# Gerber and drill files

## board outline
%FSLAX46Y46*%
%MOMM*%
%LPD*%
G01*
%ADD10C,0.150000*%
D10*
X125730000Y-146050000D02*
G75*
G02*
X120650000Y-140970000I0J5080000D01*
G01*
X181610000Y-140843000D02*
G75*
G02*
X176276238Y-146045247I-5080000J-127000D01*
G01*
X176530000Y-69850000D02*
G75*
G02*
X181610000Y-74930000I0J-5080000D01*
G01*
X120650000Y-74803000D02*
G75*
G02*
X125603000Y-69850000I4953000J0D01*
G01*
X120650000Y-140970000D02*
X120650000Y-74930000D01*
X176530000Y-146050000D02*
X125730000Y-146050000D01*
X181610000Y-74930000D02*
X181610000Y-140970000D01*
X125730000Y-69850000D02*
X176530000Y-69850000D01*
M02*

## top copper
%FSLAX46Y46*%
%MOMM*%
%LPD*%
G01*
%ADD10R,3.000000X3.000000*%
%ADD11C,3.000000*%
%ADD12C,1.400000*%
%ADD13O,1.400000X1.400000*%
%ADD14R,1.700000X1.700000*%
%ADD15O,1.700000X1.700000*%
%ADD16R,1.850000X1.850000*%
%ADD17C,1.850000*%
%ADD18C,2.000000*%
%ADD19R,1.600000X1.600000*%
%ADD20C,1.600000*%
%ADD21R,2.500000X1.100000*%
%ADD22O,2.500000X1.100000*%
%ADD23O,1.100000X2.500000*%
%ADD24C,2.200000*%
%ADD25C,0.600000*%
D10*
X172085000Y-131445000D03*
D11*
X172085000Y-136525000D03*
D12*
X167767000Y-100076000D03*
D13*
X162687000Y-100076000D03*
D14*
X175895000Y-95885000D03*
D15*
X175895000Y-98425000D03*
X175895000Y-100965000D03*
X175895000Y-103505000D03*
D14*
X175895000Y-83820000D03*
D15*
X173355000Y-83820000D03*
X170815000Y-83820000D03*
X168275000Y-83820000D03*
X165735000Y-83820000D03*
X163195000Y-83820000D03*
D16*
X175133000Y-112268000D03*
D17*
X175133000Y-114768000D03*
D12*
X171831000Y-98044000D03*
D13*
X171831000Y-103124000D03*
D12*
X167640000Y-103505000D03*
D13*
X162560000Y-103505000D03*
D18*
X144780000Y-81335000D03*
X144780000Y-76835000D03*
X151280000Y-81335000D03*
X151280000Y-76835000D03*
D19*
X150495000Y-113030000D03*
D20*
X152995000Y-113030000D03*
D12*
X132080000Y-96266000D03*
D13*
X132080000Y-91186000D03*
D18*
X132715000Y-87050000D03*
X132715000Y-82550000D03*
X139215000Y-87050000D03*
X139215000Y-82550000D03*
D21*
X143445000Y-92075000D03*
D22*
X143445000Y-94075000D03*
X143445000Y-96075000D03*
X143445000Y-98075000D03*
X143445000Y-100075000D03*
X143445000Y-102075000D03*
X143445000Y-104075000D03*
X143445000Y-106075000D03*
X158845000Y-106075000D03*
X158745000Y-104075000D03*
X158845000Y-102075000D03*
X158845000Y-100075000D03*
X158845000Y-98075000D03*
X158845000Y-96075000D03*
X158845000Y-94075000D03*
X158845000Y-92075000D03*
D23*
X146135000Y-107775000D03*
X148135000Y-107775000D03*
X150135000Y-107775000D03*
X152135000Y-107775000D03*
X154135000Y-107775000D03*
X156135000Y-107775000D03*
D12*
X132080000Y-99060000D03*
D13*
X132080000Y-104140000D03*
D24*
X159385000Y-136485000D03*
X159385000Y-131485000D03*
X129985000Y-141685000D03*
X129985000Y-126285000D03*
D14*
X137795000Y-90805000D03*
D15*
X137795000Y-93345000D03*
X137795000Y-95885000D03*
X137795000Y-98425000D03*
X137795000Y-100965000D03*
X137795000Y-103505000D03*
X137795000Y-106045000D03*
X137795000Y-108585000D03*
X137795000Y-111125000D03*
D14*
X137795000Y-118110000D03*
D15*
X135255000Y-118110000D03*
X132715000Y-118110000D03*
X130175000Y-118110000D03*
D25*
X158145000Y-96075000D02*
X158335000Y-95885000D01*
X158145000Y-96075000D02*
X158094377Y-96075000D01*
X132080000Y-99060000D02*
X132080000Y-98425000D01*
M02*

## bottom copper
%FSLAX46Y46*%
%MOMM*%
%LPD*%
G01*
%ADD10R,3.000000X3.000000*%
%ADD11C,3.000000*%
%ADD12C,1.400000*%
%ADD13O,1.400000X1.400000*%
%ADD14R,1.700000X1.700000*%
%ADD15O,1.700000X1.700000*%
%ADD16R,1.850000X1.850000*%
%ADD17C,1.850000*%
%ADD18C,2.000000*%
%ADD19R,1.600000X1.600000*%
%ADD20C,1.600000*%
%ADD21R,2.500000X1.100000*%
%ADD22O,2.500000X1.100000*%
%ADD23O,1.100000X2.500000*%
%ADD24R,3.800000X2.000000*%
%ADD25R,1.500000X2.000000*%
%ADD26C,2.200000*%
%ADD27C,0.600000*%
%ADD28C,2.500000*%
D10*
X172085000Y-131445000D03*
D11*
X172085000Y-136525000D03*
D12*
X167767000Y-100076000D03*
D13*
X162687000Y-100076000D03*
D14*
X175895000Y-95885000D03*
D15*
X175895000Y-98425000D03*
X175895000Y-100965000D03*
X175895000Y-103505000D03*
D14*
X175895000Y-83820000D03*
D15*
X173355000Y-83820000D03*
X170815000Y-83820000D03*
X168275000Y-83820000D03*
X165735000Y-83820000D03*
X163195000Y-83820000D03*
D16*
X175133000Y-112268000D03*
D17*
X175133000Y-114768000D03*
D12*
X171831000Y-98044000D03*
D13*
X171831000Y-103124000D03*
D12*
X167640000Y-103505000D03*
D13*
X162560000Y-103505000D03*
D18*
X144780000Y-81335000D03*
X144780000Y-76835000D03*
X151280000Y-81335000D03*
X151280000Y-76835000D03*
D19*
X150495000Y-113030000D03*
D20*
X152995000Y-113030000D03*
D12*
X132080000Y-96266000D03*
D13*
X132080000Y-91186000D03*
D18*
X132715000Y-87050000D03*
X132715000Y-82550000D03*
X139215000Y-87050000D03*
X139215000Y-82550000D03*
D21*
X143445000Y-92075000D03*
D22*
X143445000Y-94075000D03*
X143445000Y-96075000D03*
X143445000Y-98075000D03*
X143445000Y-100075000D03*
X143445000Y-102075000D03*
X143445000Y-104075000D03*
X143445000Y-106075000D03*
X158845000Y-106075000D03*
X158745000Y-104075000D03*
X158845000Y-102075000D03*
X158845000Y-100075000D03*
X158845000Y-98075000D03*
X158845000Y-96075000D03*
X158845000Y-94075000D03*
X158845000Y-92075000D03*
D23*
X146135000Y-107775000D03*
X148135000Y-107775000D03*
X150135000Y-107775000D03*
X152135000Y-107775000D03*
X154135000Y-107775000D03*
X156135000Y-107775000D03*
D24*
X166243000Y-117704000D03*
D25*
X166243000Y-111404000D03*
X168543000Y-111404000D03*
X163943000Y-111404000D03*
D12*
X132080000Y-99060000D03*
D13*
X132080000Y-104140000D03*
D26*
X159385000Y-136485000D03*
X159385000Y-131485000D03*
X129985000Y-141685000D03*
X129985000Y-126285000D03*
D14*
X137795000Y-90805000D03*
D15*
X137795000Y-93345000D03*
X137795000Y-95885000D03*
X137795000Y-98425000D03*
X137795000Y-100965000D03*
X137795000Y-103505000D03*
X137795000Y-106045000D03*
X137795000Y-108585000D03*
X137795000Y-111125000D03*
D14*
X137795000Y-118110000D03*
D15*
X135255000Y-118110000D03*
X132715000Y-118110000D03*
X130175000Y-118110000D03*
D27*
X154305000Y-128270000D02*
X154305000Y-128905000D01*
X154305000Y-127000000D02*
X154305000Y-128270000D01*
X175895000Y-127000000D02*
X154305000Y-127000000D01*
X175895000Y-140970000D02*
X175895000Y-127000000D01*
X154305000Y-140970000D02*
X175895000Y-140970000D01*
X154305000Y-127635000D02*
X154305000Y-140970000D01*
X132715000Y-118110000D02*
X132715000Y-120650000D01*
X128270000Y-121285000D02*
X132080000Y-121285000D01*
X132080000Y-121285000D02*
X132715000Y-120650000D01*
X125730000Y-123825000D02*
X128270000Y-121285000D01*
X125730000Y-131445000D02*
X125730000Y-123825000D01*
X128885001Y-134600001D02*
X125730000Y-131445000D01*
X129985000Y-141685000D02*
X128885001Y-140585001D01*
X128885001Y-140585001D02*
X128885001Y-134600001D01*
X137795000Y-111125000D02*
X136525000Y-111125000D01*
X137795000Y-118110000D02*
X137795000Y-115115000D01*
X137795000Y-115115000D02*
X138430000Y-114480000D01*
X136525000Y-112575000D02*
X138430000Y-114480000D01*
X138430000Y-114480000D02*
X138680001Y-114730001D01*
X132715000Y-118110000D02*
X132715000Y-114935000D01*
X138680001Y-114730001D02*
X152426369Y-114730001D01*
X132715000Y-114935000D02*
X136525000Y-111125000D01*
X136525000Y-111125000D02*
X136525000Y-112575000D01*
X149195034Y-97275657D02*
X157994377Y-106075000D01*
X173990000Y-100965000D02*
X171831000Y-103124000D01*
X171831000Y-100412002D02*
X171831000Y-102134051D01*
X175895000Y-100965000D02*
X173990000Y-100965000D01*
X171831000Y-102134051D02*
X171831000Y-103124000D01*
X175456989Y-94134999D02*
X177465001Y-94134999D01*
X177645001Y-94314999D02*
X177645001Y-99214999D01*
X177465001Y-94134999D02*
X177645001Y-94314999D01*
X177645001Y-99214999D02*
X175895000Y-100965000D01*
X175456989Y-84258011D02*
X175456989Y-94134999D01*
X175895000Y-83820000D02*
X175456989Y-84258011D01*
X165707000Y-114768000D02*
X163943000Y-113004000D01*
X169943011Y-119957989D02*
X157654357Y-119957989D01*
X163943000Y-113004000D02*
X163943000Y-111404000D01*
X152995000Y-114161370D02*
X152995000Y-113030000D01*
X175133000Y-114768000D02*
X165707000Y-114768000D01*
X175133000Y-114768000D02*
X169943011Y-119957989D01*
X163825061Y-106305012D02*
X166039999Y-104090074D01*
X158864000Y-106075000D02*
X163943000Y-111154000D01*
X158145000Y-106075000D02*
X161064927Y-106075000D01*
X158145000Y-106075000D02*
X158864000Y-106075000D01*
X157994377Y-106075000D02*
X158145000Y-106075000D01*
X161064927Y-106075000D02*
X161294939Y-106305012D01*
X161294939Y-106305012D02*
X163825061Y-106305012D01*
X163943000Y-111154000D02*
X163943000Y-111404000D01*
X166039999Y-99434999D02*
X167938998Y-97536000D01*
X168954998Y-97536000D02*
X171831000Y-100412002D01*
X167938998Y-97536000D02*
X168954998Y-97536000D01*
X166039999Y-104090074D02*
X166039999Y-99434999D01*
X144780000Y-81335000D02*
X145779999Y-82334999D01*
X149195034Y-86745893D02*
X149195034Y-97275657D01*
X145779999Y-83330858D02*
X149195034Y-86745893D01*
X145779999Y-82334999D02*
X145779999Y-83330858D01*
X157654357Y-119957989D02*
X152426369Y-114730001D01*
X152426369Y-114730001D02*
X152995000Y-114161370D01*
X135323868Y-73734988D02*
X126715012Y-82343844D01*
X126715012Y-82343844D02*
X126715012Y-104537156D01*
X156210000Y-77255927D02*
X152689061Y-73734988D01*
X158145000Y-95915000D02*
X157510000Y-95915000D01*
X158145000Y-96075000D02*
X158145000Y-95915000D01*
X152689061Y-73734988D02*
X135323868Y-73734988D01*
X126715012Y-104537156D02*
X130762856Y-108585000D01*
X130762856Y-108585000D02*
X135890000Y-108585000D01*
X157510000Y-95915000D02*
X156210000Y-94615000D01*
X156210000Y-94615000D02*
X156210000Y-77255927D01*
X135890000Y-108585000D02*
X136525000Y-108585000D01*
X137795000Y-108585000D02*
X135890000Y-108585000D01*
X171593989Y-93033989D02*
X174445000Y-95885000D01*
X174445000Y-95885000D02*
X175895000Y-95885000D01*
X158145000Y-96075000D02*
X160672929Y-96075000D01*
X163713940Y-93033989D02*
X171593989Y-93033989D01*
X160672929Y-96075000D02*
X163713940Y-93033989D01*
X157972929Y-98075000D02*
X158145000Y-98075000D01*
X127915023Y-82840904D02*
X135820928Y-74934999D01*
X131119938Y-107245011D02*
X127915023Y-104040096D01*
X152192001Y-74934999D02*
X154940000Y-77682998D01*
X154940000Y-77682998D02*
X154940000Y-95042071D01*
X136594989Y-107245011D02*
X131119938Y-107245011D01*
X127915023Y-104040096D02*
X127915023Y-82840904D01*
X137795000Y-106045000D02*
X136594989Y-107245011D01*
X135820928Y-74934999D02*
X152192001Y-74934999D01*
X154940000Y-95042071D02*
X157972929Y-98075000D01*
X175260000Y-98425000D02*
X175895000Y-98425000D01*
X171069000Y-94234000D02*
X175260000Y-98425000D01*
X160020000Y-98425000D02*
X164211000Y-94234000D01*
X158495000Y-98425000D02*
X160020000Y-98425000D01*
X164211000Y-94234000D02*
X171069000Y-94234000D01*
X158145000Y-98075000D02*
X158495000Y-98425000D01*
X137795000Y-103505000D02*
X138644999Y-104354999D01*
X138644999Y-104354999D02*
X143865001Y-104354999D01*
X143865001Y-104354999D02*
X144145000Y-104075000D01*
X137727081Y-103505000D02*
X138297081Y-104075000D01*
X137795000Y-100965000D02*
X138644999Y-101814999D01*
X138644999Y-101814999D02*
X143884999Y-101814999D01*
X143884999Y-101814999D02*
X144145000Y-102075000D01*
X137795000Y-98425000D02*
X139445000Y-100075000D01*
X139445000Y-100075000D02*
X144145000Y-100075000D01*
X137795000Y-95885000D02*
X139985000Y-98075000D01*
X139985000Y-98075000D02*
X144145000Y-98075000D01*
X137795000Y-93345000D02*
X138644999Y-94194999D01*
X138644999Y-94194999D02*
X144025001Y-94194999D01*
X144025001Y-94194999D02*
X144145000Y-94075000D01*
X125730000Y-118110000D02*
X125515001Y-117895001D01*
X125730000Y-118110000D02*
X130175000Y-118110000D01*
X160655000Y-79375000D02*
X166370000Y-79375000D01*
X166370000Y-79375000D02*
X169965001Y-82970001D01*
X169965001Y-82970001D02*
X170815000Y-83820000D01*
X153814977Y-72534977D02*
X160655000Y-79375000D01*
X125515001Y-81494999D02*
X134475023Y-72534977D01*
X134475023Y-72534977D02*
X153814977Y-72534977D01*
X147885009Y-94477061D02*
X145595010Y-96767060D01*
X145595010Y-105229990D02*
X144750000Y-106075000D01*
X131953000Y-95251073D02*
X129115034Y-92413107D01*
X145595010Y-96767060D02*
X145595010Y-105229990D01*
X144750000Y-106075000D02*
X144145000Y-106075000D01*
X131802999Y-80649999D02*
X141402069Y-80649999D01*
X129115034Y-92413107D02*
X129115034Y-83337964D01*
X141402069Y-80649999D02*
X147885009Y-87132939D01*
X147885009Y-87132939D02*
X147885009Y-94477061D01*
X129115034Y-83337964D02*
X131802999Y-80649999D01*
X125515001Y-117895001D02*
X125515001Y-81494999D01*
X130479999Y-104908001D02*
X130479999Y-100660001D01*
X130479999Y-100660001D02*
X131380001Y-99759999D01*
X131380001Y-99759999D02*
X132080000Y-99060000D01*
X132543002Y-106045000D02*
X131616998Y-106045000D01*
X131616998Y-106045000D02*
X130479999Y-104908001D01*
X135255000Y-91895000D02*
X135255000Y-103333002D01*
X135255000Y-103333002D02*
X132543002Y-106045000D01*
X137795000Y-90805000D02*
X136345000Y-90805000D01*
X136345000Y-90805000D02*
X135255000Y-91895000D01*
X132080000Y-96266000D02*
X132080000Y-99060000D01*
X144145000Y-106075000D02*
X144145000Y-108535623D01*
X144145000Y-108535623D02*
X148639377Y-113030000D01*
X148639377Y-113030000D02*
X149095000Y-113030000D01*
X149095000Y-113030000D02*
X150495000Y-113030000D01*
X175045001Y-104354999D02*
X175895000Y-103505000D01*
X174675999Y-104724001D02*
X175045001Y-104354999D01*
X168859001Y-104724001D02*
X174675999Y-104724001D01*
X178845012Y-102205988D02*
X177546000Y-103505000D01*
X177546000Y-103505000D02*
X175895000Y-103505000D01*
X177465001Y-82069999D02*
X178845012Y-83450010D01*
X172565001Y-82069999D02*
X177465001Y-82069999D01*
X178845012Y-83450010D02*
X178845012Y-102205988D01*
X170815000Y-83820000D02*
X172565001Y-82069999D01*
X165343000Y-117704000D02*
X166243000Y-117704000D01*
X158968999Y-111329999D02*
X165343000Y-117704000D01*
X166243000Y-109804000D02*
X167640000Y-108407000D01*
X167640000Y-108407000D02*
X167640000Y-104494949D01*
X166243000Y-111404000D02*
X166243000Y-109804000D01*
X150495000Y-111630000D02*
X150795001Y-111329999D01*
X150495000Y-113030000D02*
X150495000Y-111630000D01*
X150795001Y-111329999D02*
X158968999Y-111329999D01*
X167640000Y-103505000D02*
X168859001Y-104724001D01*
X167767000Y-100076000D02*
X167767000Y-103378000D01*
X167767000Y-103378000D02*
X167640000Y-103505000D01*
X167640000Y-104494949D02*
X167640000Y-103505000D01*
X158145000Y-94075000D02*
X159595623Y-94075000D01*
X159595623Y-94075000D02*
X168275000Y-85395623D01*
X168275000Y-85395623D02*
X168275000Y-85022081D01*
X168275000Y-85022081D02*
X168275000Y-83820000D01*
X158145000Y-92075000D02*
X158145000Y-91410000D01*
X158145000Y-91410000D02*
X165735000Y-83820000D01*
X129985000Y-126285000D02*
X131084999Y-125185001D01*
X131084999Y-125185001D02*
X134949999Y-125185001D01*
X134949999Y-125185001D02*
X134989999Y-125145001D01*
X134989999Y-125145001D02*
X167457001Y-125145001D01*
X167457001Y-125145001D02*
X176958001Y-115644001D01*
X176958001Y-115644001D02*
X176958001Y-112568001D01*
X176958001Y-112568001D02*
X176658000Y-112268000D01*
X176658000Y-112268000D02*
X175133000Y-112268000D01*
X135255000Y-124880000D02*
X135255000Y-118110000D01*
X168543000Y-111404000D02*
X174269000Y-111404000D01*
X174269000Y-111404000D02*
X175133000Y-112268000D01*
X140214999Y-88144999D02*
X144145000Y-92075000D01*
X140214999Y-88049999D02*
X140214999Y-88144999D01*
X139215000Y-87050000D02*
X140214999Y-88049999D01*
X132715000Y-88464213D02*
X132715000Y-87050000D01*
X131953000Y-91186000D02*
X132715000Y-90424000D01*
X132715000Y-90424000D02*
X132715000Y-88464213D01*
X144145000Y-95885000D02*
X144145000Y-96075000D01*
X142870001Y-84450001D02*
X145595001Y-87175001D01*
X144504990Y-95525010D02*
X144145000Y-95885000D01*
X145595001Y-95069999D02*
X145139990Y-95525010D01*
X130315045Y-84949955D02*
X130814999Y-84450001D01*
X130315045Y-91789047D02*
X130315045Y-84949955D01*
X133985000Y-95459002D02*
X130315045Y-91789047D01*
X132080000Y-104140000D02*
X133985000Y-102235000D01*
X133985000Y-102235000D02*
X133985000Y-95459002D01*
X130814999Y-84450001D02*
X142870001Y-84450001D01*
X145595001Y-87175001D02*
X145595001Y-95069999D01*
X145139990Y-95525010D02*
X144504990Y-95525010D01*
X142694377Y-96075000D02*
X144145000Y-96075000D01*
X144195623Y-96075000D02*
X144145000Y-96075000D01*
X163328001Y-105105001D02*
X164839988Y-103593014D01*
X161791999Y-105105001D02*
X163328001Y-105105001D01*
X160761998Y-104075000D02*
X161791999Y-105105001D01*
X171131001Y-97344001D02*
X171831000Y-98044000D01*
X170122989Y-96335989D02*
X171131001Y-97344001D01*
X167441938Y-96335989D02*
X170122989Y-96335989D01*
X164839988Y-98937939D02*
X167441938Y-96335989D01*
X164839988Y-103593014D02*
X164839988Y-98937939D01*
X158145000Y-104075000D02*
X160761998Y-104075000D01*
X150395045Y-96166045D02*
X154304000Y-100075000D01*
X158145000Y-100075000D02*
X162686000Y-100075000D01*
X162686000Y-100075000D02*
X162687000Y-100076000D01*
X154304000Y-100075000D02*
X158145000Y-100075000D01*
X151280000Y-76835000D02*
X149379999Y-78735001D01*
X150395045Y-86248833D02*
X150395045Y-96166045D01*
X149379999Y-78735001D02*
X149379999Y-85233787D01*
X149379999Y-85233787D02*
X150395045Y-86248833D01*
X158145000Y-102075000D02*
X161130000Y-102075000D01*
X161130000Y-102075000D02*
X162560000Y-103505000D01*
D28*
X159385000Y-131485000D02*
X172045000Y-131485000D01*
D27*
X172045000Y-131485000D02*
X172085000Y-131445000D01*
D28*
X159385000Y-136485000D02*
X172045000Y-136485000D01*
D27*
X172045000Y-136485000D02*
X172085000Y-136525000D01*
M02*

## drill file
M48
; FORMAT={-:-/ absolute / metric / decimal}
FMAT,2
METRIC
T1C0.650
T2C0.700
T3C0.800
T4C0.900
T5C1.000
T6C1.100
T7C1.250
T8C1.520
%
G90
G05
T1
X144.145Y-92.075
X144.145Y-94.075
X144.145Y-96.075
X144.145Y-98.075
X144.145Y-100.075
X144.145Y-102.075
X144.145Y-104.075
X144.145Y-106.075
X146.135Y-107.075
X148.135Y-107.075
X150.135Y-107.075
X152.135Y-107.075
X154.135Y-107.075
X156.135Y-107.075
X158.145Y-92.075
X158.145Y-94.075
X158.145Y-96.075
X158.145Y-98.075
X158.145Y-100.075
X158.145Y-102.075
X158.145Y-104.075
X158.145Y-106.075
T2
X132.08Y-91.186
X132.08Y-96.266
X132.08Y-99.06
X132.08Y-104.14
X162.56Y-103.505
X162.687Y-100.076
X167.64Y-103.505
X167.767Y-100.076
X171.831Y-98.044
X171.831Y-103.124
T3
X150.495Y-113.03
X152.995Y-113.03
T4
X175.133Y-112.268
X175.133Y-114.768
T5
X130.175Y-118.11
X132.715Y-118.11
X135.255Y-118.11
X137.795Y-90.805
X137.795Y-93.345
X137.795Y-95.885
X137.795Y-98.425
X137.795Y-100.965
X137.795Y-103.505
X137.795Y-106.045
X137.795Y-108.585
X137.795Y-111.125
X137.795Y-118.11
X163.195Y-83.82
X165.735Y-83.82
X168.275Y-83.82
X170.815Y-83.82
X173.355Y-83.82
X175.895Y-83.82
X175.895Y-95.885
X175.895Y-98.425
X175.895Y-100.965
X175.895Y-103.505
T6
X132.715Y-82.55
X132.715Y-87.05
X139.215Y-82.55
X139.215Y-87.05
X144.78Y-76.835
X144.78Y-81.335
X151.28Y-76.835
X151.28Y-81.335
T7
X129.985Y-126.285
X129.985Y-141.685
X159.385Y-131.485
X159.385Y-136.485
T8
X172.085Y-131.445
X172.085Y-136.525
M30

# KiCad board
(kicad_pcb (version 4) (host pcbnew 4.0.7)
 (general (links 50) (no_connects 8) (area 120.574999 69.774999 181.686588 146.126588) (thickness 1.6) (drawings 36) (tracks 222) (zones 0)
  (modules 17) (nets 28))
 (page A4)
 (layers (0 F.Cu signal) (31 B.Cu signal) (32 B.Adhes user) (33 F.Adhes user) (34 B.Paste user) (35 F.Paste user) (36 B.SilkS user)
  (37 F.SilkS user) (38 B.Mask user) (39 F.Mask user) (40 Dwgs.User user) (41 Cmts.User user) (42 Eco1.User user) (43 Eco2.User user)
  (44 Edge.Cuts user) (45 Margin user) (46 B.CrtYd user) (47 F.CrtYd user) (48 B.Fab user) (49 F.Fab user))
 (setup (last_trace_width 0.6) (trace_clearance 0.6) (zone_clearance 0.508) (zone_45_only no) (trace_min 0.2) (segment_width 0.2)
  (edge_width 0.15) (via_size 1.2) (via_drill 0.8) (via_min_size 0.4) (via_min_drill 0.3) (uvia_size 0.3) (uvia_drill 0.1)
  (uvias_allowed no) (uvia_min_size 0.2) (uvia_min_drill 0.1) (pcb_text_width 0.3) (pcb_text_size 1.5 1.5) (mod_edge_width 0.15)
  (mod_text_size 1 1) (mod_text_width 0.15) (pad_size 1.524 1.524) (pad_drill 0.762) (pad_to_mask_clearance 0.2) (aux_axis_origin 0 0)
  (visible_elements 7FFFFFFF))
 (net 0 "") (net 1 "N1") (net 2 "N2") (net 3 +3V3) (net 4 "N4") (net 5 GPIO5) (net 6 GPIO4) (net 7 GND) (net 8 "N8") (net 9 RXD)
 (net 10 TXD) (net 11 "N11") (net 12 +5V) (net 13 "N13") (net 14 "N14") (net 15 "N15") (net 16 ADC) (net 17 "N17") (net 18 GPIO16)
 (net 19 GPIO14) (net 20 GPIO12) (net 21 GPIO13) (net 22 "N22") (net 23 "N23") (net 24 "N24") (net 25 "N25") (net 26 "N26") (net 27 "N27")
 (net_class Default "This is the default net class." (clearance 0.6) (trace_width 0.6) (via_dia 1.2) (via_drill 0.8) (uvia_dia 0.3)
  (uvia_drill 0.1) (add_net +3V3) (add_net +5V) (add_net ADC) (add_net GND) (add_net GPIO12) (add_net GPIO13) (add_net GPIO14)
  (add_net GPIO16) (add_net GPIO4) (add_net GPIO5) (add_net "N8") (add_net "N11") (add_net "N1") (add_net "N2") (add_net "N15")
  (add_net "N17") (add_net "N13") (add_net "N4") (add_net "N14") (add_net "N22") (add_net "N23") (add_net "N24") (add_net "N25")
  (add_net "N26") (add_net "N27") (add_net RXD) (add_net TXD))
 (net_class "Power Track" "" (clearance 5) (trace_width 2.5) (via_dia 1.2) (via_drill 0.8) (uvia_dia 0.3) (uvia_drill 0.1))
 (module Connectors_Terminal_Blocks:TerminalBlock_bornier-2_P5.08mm (layer F.Cu) (at 172.085 131.445 270)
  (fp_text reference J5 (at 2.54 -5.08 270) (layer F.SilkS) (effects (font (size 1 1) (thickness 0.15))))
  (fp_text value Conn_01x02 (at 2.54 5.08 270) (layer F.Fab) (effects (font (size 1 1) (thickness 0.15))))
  (pad 1 thru_hole rect (at 0 0 270) (size 3 3) (drill 1.52) (layers *.Cu *.Mask) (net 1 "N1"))
  (pad 2 thru_hole circle (at 5.08 0 270) (size 3 3) (drill 1.52) (layers *.Cu *.Mask) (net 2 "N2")))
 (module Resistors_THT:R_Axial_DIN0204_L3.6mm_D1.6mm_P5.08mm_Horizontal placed (layer F.Cu) (at 167.767 100.076 180)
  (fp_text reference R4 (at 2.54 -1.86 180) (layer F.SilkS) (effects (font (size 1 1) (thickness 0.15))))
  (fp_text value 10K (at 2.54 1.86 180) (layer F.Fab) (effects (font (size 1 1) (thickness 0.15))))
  (pad 1 thru_hole circle (at 0 0 180) (size 1.4 1.4) (drill 0.7) (layers *.Cu *.Mask) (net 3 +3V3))
  (pad 2 thru_hole oval (at 5.08 0 180) (size 1.4 1.4) (drill 0.7) (layers *.Cu *.Mask) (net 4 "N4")))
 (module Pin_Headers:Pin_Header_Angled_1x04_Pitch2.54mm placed (layer F.Cu) (at 175.895 95.885)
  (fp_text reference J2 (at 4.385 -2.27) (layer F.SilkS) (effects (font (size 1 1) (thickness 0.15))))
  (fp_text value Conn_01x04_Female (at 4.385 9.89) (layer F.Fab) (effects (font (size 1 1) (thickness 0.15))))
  (pad 1 thru_hole rect (at 0 0) (size 1.7 1.7) (drill 1) (layers *.Cu *.Mask) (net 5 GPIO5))
  (pad 2 thru_hole oval (at 0 2.54) (size 1.7 1.7) (drill 1) (layers *.Cu *.Mask) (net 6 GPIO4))
  (pad 3 thru_hole oval (at 0 5.08) (size 1.7 1.7) (drill 1) (layers *.Cu *.Mask) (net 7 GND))
  (pad 4 thru_hole oval (at 0 7.62) (size 1.7 1.7) (drill 1) (layers *.Cu *.Mask) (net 3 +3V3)))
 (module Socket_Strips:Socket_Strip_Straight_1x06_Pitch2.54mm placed (layer F.Cu) (at 175.895 83.82 270)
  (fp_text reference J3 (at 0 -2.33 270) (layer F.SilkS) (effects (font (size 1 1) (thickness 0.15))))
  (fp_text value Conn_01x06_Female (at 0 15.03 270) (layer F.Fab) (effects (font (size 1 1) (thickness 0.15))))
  (pad 1 thru_hole rect (at 0 0 270) (size 1.7 1.7) (drill 1) (layers *.Cu *.Mask) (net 7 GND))
  (pad 2 thru_hole oval (at 0 2.54 270) (size 1.7 1.7) (drill 1) (layers *.Cu *.Mask) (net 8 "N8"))
  (pad 3 thru_hole oval (at 0 5.08 270) (size 1.7 1.7) (drill 1) (layers *.Cu *.Mask) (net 3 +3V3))
  (pad 4 thru_hole oval (at 0 7.62 270) (size 1.7 1.7) (drill 1) (layers *.Cu *.Mask) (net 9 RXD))
  (pad 5 thru_hole oval (at 0 10.16 270) (size 1.7 1.7) (drill 1) (layers *.Cu *.Mask) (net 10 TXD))
  (pad 6 thru_hole oval (at 0 12.7 270) (size 1.7 1.7) (drill 1) (layers *.Cu *.Mask) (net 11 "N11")))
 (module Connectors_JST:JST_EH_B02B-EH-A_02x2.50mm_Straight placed (layer F.Cu) (at 175.133 112.268 270)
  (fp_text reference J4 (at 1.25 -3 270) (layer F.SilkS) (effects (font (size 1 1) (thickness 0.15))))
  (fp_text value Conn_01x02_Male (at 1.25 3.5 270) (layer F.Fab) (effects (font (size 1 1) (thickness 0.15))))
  (pad 1 thru_hole rect (at 0 0 270) (size 1.85 1.85) (drill 0.9) (layers *.Cu *.Mask) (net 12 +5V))
  (pad 2 thru_hole circle (at 2.5 0 270) (size 1.85 1.85) (drill 0.9) (layers *.Cu *.Mask) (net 7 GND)))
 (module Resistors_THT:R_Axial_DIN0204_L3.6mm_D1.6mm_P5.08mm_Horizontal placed (layer F.Cu) (at 171.831 98.044 270)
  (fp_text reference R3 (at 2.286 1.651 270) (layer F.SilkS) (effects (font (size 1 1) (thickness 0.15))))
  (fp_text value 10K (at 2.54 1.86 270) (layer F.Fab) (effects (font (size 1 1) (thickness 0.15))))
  (pad 1 thru_hole circle (at 0 0 270) (size 1.4 1.4) (drill 0.7) (layers *.Cu *.Mask) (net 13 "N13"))
  (pad 2 thru_hole oval (at 5.08 0 270) (size 1.4 1.4) (drill 0.7) (layers *.Cu *.Mask) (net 7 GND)))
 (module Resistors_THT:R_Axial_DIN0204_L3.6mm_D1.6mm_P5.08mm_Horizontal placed (layer F.Cu) (at 167.64 103.505 180)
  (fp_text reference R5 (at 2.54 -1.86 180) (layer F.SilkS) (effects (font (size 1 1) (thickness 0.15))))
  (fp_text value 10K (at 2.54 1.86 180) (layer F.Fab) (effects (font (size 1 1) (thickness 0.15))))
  (pad 1 thru_hole circle (at 0 0 180) (size 1.4 1.4) (drill 0.7) (layers *.Cu *.Mask) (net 3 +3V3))
  (pad 2 thru_hole oval (at 5.08 0 180) (size 1.4 1.4) (drill 0.7) (layers *.Cu *.Mask) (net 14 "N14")))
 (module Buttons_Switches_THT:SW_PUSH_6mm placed (layer F.Cu) (at 144.78 76.835)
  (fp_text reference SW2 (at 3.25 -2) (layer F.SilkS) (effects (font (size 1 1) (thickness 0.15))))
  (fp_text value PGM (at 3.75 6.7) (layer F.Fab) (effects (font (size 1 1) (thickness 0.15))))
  (pad 2 thru_hole circle (at 0 4.5 90) (size 2 2) (drill 1.1) (layers *.Cu *.Mask) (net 7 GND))
  (pad 1 thru_hole circle (at 0 0 90) (size 2 2) (drill 1.1) (layers *.Cu *.Mask) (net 4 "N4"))
  (pad 2 thru_hole circle (at 6.5 4.5 90) (size 2 2) (drill 1.1) (layers *.Cu *.Mask) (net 7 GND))
  (pad 1 thru_hole circle (at 6.5 0 90) (size 2 2) (drill 1.1) (layers *.Cu *.Mask) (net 4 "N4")))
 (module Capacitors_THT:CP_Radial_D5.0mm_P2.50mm (layer F.Cu) (at 150.495 113.03)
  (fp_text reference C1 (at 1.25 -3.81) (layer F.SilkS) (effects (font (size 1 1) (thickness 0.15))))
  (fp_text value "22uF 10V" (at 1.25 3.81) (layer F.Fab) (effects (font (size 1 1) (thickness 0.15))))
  (pad 1 thru_hole rect (at 0 0) (size 1.6 1.6) (drill 0.8) (layers *.Cu *.Mask) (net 3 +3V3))
  (pad 2 thru_hole circle (at 2.5 0) (size 1.6 1.6) (drill 0.8) (layers *.Cu *.Mask) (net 7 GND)))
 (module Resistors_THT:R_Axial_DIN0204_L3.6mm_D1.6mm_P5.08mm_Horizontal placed (layer F.Cu) (at 132.08 96.266 90)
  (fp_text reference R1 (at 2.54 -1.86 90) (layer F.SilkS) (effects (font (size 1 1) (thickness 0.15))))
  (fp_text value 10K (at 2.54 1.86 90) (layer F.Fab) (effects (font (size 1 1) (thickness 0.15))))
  (pad 1 thru_hole circle (at 0 0 90) (size 1.4 1.4) (drill 0.7) (layers *.Cu *.Mask) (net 3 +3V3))
  (pad 2 thru_hole oval (at 5.08 0 90) (size 1.4 1.4) (drill 0.7) (layers *.Cu *.Mask) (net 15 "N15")))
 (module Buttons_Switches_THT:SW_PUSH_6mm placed (layer F.Cu) (at 132.715 82.55)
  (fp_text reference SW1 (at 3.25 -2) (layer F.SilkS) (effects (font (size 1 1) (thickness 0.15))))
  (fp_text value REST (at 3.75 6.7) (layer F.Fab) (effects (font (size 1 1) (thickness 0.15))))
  (pad 2 thru_hole circle (at 0 4.5 90) (size 2 2) (drill 1.1) (layers *.Cu *.Mask) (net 15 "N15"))
  (pad 1 thru_hole circle (at 0 0 90) (size 2 2) (drill 1.1) (layers *.Cu *.Mask) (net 7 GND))
  (pad 2 thru_hole circle (at 6.5 4.5 90) (size 2 2) (drill 1.1) (layers *.Cu *.Mask) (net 15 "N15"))
  (pad 1 thru_hole circle (at 6.5 0 90) (size 2 2) (drill 1.1) (layers *.Cu *.Mask) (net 7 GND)))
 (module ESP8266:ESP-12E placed (layer F.Cu) (at 144.145 92.075)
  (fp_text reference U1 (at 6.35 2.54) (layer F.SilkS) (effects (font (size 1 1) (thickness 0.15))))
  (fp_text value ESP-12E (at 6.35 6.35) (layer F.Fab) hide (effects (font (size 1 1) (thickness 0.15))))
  (pad 1 thru_hole rect (at 0 0) (size 2.5 1.1) (drill 0.65 (offset -0.7 0)) (layers *.Cu *.Mask F.SilkS) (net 15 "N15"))
  (pad 2 thru_hole oval (at 0 2) (size 2.5 1.1) (drill 0.65 (offset -0.7 0)) (layers *.Cu *.Mask F.SilkS) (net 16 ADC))
  (pad 3 thru_hole oval (at 0 4) (size 2.5 1.1) (drill 0.65 (offset -0.7 0)) (layers *.Cu *.Mask F.SilkS) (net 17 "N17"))
  (pad 4 thru_hole oval (at 0 6) (size 2.5 1.1) (drill 0.65 (offset -0.7 0)) (layers *.Cu *.Mask F.SilkS) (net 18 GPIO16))
  (pad 5 thru_hole oval (at 0 8) (size 2.5 1.1) (drill 0.65 (offset -0.7 0)) (layers *.Cu *.Mask F.SilkS) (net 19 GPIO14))
  (pad 6 thru_hole oval (at 0 10) (size 2.5 1.1) (drill 0.65 (offset -0.7 0)) (layers *.Cu *.Mask F.SilkS) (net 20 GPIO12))
  (pad 7 thru_hole oval (at 0 12) (size 2.5 1.1) (drill 0.65 (offset -0.7 0)) (layers *.Cu *.Mask F.SilkS) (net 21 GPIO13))
  (pad 8 thru_hole oval (at 0 14) (size 2.5 1.1) (drill 0.65 (offset -0.7 0)) (layers *.Cu *.Mask F.SilkS) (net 3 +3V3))
  (pad 9 thru_hole oval (at 14 14) (size 2.5 1.1) (drill 0.65 (offset 0.7 0)) (layers *.Cu *.Mask F.SilkS) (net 7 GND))
  (pad 10 thru_hole oval (at 14 12) (size 2.5 1.1) (drill 0.65 (offset 0.6 0)) (layers *.Cu *.Mask F.SilkS) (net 13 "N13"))
  (pad 11 thru_hole oval (at 14 10) (size 2.5 1.1) (drill 0.65 (offset 0.7 0)) (layers *.Cu *.Mask F.SilkS) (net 14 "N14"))
  (pad 12 thru_hole oval (at 14 8) (size 2.5 1.1) (drill 0.65 (offset 0.7 0)) (layers *.Cu *.Mask F.SilkS) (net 4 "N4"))
  (pad 13 thru_hole oval (at 14 6) (size 2.5 1.1) (drill 0.65 (offset 0.7 0)) (layers *.Cu *.Mask F.SilkS) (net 6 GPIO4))
  (pad 14 thru_hole oval (at 14 4) (size 2.5 1.1) (drill 0.65 (offset 0.7 0)) (layers *.Cu *.Mask F.SilkS) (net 5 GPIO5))
  (pad 15 thru_hole oval (at 14 2) (size 2.5 1.1) (drill 0.65 (offset 0.7 0)) (layers *.Cu *.Mask F.SilkS) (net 9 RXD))
  (pad 16 thru_hole oval (at 14 0) (size 2.5 1.1) (drill 0.65 (offset 0.7 0)) (layers *.Cu *.Mask F.SilkS) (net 10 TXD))
  (pad 17 thru_hole oval (at 1.99 15 90) (size 2.5 1.1) (drill 0.65 (offset -0.7 0)) (layers *.Cu *.Mask F.SilkS) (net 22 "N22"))
  (pad 18 thru_hole oval (at 3.99 15 90) (size 2.5 1.1) (drill 0.65 (offset -0.7 0)) (layers *.Cu *.Mask F.SilkS) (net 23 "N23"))
  (pad 19 thru_hole oval (at 5.99 15 90) (size 2.5 1.1) (drill 0.65 (offset -0.7 0)) (layers *.Cu *.Mask F.SilkS) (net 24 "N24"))
  (pad 20 thru_hole oval (at 7.99 15 90) (size 2.5 1.1) (drill 0.65 (offset -0.7 0)) (layers *.Cu *.Mask F.SilkS) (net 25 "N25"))
  (pad 21 thru_hole oval (at 9.99 15 90) (size 2.5 1.1) (drill 0.65 (offset -0.7 0)) (layers *.Cu *.Mask F.SilkS) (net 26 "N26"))
  (pad 22 thru_hole oval (at 11.99 15 90) (size 2.5 1.1) (drill 0.65 (offset -0.7 0)) (layers *.Cu *.Mask F.SilkS) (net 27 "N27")))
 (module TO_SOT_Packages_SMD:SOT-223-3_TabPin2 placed (layer B.Cu) (at 166.243 114.554 270)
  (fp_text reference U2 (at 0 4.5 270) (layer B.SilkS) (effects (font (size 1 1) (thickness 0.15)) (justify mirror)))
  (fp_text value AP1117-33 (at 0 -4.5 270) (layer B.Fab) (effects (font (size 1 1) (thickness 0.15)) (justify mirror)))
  (pad 2 smd rect (at 3.15 0 270) (size 2 3.8) (layers B.Cu B.Paste B.Mask) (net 3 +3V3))
  (pad 2 smd rect (at -3.15 0 270) (size 2 1.5) (layers B.Cu B.Paste B.Mask) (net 3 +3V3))
  (pad 3 smd rect (at -3.15 -2.3 270) (size 2 1.5) (layers B.Cu B.Paste B.Mask) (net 12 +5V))
  (pad 1 smd rect (at -3.15 2.3 270) (size 2 1.5) (layers B.Cu B.Paste B.Mask) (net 7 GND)))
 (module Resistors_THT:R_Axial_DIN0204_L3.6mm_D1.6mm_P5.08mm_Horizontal (layer F.Cu) (at 132.08 99.06 270)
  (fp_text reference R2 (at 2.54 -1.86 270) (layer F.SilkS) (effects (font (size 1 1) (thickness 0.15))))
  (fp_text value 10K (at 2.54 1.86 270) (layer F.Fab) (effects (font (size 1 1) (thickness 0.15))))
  (pad 1 thru_hole circle (at 0 0 270) (size 1.4 1.4) (drill 0.7) (layers *.Cu *.Mask) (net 3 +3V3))
  (pad 2 thru_hole oval (at 5.08 0 270) (size 1.4 1.4) (drill 0.7) (layers *.Cu *.Mask) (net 17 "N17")))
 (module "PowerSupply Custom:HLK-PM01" (layer F.Cu) (at 144.685 133.985 180)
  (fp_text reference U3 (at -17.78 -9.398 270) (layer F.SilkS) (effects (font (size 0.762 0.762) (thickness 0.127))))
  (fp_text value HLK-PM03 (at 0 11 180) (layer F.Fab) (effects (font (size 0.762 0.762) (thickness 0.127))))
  (pad 1 thru_hole circle (at -14.7 -2.5 180) (size 2.2 2.2) (drill 1.25) (layers *.Cu *.Mask) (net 2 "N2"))
  (pad 2 thru_hole circle (at -14.7 2.5 180) (size 2.2 2.2) (drill 1.25) (layers *.Cu *.Mask) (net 1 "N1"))
  (pad 3 thru_hole circle (at 14.7 -7.7 180) (size 2.2 2.2) (drill 1.25) (layers *.Cu *.Mask) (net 7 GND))
  (pad 4 thru_hole circle (at 14.7 7.7 180) (size 2.2 2.2) (drill 1.25) (layers *.Cu *.Mask) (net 12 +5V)))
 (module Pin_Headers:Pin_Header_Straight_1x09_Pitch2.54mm (layer F.Cu) (at 137.795 90.805)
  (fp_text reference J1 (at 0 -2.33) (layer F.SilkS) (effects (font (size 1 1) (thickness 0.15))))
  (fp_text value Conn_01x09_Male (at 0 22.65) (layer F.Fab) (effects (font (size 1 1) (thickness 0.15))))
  (pad 1 thru_hole rect (at 0 0) (size 1.7 1.7) (drill 1) (layers *.Cu *.Mask) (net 3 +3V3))
  (pad 2 thru_hole oval (at 0 2.54) (size 1.7 1.7) (drill 1) (layers *.Cu *.Mask) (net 16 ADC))
  (pad 3 thru_hole oval (at 0 5.08) (size 1.7 1.7) (drill 1) (layers *.Cu *.Mask) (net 18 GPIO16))
  (pad 4 thru_hole oval (at 0 7.62) (size 1.7 1.7) (drill 1) (layers *.Cu *.Mask) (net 19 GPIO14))
  (pad 5 thru_hole oval (at 0 10.16) (size 1.7 1.7) (drill 1) (layers *.Cu *.Mask) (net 20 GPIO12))
  (pad 6 thru_hole oval (at 0 12.7) (size 1.7 1.7) (drill 1) (layers *.Cu *.Mask) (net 21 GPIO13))
  (pad 7 thru_hole oval (at 0 15.24) (size 1.7 1.7) (drill 1) (layers *.Cu *.Mask) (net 6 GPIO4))
  (pad 8 thru_hole oval (at 0 17.78) (size 1.7 1.7) (drill 1) (layers *.Cu *.Mask) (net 5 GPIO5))
  (pad 9 thru_hole oval (at 0 20.32) (size 1.7 1.7) (drill 1) (layers *.Cu *.Mask) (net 7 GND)))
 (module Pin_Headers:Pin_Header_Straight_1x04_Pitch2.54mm (layer F.Cu) (at 137.795 118.11 270)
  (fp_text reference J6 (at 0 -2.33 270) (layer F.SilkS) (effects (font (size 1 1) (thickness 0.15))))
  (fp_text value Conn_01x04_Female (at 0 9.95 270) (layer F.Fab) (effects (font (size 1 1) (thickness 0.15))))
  (pad 1 thru_hole rect (at 0 0 270) (size 1.7 1.7) (drill 1) (layers *.Cu *.Mask) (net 7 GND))
  (pad 2 thru_hole oval (at 0 2.54 270) (size 1.7 1.7) (drill 1) (layers *.Cu *.Mask) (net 12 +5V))
  (pad 3 thru_hole oval (at 0 5.08 270) (size 1.7 1.7) (drill 1) (layers *.Cu *.Mask) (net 7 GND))
  (pad 4 thru_hole oval (at 0 7.62 270) (size 1.7 1.7) (drill 1) (layers *.Cu *.Mask) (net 3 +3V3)))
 (gr_arc (start 125.73 140.97) (end 125.73 146.05) (angle 90) (layer Edge.Cuts) (width 0.15))
 (gr_arc (start 176.53 140.97) (end 181.61 140.843) (angle 94.29450141) (layer Edge.Cuts) (width 0.15))
 (gr_arc (start 176.53 74.93) (end 176.53 69.85) (angle 90) (layer Edge.Cuts) (width 0.15))
 (gr_arc (start 125.603 74.803) (end 120.65 74.803) (angle 90) (layer Edge.Cuts) (width 0.15))
 (gr_line (start 120.65 140.97) (end 120.65 74.93) (layer Edge.Cuts) (width 0.15))
 (gr_line (start 176.53 146.05) (end 125.73 146.05) (layer Edge.Cuts) (width 0.15))
 (gr_line (start 181.61 74.93) (end 181.61 140.97) (layer Edge.Cuts) (width 0.15))
 (gr_line (start 125.73 69.85) (end 176.53 69.85) (layer Edge.Cuts) (width 0.15))
 (segment (start 154.305 128.27) (end 154.305 128.905) (width 0.6) (layer B.Cu) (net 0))
 (segment (start 154.305 127) (end 154.305 128.27) (width 0.6) (layer B.Cu) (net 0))
 (segment (start 175.895 127) (end 154.305 127) (width 0.6) (layer B.Cu) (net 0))
 (segment (start 175.895 140.97) (end 175.895 127) (width 0.6) (layer B.Cu) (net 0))
 (segment (start 154.305 140.97) (end 175.895 140.97) (width 0.6) (layer B.Cu) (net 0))
 (segment (start 154.305 127.635) (end 154.305 140.97) (width 0.6) (layer B.Cu) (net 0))
 (segment (start 132.715 118.11) (end 132.715 120.65) (width 0.6) (layer B.Cu) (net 7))
 (segment (start 128.27 121.285) (end 132.08 121.285) (width 0.6) (layer B.Cu) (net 7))
 (segment (start 132.08 121.285) (end 132.715 120.65) (width 0.6) (layer B.Cu) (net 7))
 (segment (start 125.73 123.825) (end 128.27 121.285) (width 0.6) (layer B.Cu) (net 7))
 (segment (start 125.73 131.445) (end 125.73 123.825) (width 0.6) (layer B.Cu) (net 7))
 (segment (start 128.885001 134.600001) (end 125.73 131.445) (width 0.6) (layer B.Cu) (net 7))
 (segment (start 129.985 141.685) (end 128.885001 140.585001) (width 0.6) (layer B.Cu) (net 7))
 (segment (start 128.885001 140.585001) (end 128.885001 134.600001) (width 0.6) (layer B.Cu) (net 7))
 (segment (start 137.795 111.125) (end 136.525 111.125) (width 0.6) (layer B.Cu) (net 7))
 (segment (start 137.795 118.11) (end 137.795 115.115) (width 0.6) (layer B.Cu) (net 7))
 (segment (start 137.795 115.115) (end 138.43 114.48) (width 0.6) (layer B.Cu) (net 7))
 (segment (start 136.525 112.575) (end 138.43 114.48) (width 0.6) (layer B.Cu) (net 7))
 (segment (start 138.43 114.48) (end 138.680001 114.730001) (width 0.6) (layer B.Cu) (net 7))
 (segment (start 132.715 118.11) (end 132.715 114.935) (width 0.6) (layer B.Cu) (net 7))
 (segment (start 138.680001 114.730001) (end 152.426369 114.730001) (width 0.6) (layer B.Cu) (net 7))
 (segment (start 132.715 114.935) (end 136.525 111.125) (width 0.6) (layer B.Cu) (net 7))
 (segment (start 136.525 111.125) (end 136.525 112.575) (width 0.6) (layer B.Cu) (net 7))
 (segment (start 149.195034 97.275657) (end 157.994377 106.075) (width 0.6) (layer B.Cu) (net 7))
 (segment (start 173.99 100.965) (end 171.831 103.124) (width 0.6) (layer B.Cu) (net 7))
 (segment (start 171.831 100.412002) (end 171.831 102.134051) (width 0.6) (layer B.Cu) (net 7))
 (segment (start 175.895 100.965) (end 173.99 100.965) (width 0.6) (layer B.Cu) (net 7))
 (segment (start 171.831 102.134051) (end 171.831 103.124) (width 0.6) (layer B.Cu) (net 7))
 (segment (start 175.456989 94.134999) (end 177.465001 94.134999) (width 0.6) (layer B.Cu) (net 7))
 (segment (start 177.645001 94.314999) (end 177.645001 99.214999) (width 0.6) (layer B.Cu) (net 7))
 (segment (start 177.465001 94.134999) (end 177.645001 94.314999) (width 0.6) (layer B.Cu) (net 7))
 (segment (start 177.645001 99.214999) (end 175.895 100.965) (width 0.6) (layer B.Cu) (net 7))
 (segment (start 175.456989 84.258011) (end 175.456989 94.134999) (width 0.6) (layer B.Cu) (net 7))
 (segment (start 175.895 83.82) (end 175.456989 84.258011) (width 0.6) (layer B.Cu) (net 7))
 (segment (start 165.707 114.768) (end 163.943 113.004) (width 0.6) (layer B.Cu) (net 7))
 (segment (start 169.943011 119.957989) (end 157.654357 119.957989) (width 0.6) (layer B.Cu) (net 7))
 (segment (start 163.943 113.004) (end 163.943 111.404) (width 0.6) (layer B.Cu) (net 7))
 (segment (start 152.995 114.16137) (end 152.995 113.03) (width 0.6) (layer B.Cu) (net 7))
 (segment (start 175.133 114.768) (end 165.707 114.768) (width 0.6) (layer B.Cu) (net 7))
 (segment (start 175.133 114.768) (end 169.943011 119.957989) (width 0.6) (layer B.Cu) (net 7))
 (segment (start 163.825061 106.305012) (end 166.039999 104.090074) (width 0.6) (layer B.Cu) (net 7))
 (segment (start 158.864 106.075) (end 163.943 111.154) (width 0.6) (layer B.Cu) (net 7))
 (segment (start 158.145 106.075) (end 161.064927 106.075) (width 0.6) (layer B.Cu) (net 7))
 (segment (start 158.145 106.075) (end 158.864 106.075) (width 0.6) (layer B.Cu) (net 7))
 (segment (start 157.994377 106.075) (end 158.145 106.075) (width 0.6) (layer B.Cu) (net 7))
 (segment (start 161.064927 106.075) (end 161.294939 106.305012) (width 0.6) (layer B.Cu) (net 7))
 (segment (start 161.294939 106.305012) (end 163.825061 106.305012) (width 0.6) (layer B.Cu) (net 7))
 (segment (start 163.943 111.154) (end 163.943 111.404) (width 0.6) (layer B.Cu) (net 7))
 (segment (start 166.039999 99.434999) (end 167.938998 97.536) (width 0.6) (layer B.Cu) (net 7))
 (segment (start 168.954998 97.536) (end 171.831 100.412002) (width 0.6) (layer B.Cu) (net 7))
 (segment (start 167.938998 97.536) (end 168.954998 97.536) (width 0.6) (layer B.Cu) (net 7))
 (segment (start 166.039999 104.090074) (end 166.039999 99.434999) (width 0.6) (layer B.Cu) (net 7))
 (segment (start 144.78 81.335) (end 145.779999 82.334999) (width 0.6) (layer B.Cu) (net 7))
 (segment (start 149.195034 86.745893) (end 149.195034 97.275657) (width 0.6) (layer B.Cu) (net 7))
 (segment (start 145.779999 83.330858) (end 149.195034 86.745893) (width 0.6) (layer B.Cu) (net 7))
 (segment (start 145.779999 82.334999) (end 145.779999 83.330858) (width 0.6) (layer B.Cu) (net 7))
 (segment (start 157.654357 119.957989) (end 152.426369 114.730001) (width 0.6) (layer B.Cu) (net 7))
 (segment (start 152.426369 114.730001) (end 152.995 114.16137) (width 0.6) (layer B.Cu) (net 7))
 (segment (start 135.323868 73.734988) (end 126.715012 82.343844) (width 0.6) (layer B.Cu) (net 5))
 (segment (start 126.715012 82.343844) (end 126.715012 104.537156) (width 0.6) (layer B.Cu) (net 5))
 (segment (start 156.21 77.255927) (end 152.689061 73.734988) (width 0.6) (layer B.Cu) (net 5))
 (segment (start 158.145 95.915) (end 157.51 95.915) (width 0.6) (layer B.Cu) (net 5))
 (segment (start 158.145 96.075) (end 158.145 95.915) (width 0.6) (layer B.Cu) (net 5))
 (segment (start 152.689061 73.734988) (end 135.323868 73.734988) (width 0.6) (layer B.Cu) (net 5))
 (segment (start 126.715012 104.537156) (end 130.762856 108.585) (width 0.6) (layer B.Cu) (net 5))
 (segment (start 130.762856 108.585) (end 135.89 108.585) (width 0.6) (layer B.Cu) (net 5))
 (segment (start 157.51 95.915) (end 156.21 94.615) (width 0.6) (layer B.Cu) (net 5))
 (segment (start 156.21 94.615) (end 156.21 77.255927) (width 0.6) (layer B.Cu) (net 5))
 (segment (start 135.89 108.585) (end 136.525 108.585) (width 0.6) (layer B.Cu) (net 5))
 (segment (start 137.795 108.585) (end 135.89 108.585) (width 0.6) (layer B.Cu) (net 5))
 (segment (start 158.145 96.075) (end 158.335 95.885) (width 0.6) (layer F.Cu) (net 5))
 (segment (start 158.145 96.075) (end 158.094377 96.075) (width 0.6) (layer F.Cu) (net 5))
 (segment (start 171.593989 93.033989) (end 174.445 95.885) (width 0.6) (layer B.Cu) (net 5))
 (segment (start 174.445 95.885) (end 175.895 95.885) (width 0.6) (layer B.Cu) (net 5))
 (segment (start 158.145 96.075) (end 160.672929 96.075) (width 0.6) (layer B.Cu) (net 5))
 (segment (start 163.71394 93.033989) (end 171.593989 93.033989) (width 0.6) (layer B.Cu) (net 5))
 (segment (start 160.672929 96.075) (end 163.71394 93.033989) (width 0.6) (layer B.Cu) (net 5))
 (segment (start 157.972929 98.075) (end 158.145 98.075) (width 0.6) (layer B.Cu) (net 6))
 (segment (start 127.915023 82.840904) (end 135.820928 74.934999) (width 0.6) (layer B.Cu) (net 6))
 (segment (start 131.119938 107.245011) (end 127.915023 104.040096) (width 0.6) (layer B.Cu) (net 6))
 (segment (start 152.192001 74.934999) (end 154.94 77.682998) (width 0.6) (layer B.Cu) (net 6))
 (segment (start 154.94 77.682998) (end 154.94 95.042071) (width 0.6) (layer B.Cu) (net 6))
 (segment (start 136.594989 107.245011) (end 131.119938 107.245011) (width 0.6) (layer B.Cu) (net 6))
 (segment (start 127.915023 104.040096) (end 127.915023 82.840904) (width 0.6) (layer B.Cu) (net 6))
 (segment (start 137.795 106.045) (end 136.594989 107.245011) (width 0.6) (layer B.Cu) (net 6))
 (segment (start 135.820928 74.934999) (end 152.192001 74.934999) (width 0.6) (layer B.Cu) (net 6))
 (segment (start 154.94 95.042071) (end 157.972929 98.075) (width 0.6) (layer B.Cu) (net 6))
 (segment (start 175.26 98.425) (end 175.895 98.425) (width 0.6) (layer B.Cu) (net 6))
 (segment (start 171.069 94.234) (end 175.26 98.425) (width 0.6) (layer B.Cu) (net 6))
 (segment (start 160.02 98.425) (end 164.211 94.234) (width 0.6) (layer B.Cu) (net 6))
 (segment (start 158.495 98.425) (end 160.02 98.425) (width 0.6) (layer B.Cu) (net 6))
 (segment (start 164.211 94.234) (end 171.069 94.234) (width 0.6) (layer B.Cu) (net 6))
 (segment (start 158.145 98.075) (end 158.495 98.425) (width 0.6) (layer B.Cu) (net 6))
 (segment (start 137.795 103.505) (end 138.644999 104.354999) (width 0.6) (layer B.Cu) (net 21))
 (segment (start 138.644999 104.354999) (end 143.865001 104.354999) (width 0.6) (layer B.Cu) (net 21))
 (segment (start 143.865001 104.354999) (end 144.145 104.075) (width 0.6) (layer B.Cu) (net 21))
 (segment (start 137.727081 103.505) (end 138.297081 104.075) (width 0.6) (layer B.Cu) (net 21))
 (segment (start 137.795 100.965) (end 138.644999 101.814999) (width 0.6) (layer B.Cu) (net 20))
 (segment (start 138.644999 101.814999) (end 143.884999 101.814999) (width 0.6) (layer B.Cu) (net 20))
 (segment (start 143.884999 101.814999) (end 144.145 102.075) (width 0.6) (layer B.Cu) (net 20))
 (segment (start 137.795 98.425) (end 139.445 100.075) (width 0.6) (layer B.Cu) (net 19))
 (segment (start 139.445 100.075) (end 144.145 100.075) (width 0.6) (layer B.Cu) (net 19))
 (segment (start 137.795 95.885) (end 139.985 98.075) (width 0.6) (layer B.Cu) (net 18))
 (segment (start 139.985 98.075) (end 144.145 98.075) (width 0.6) (layer B.Cu) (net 18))
 (segment (start 137.795 93.345) (end 138.644999 94.194999) (width 0.6) (layer B.Cu) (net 16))
 (segment (start 138.644999 94.194999) (end 144.025001 94.194999) (width 0.6) (layer B.Cu) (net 16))
 (segment (start 144.025001 94.194999) (end 144.145 94.075) (width 0.6) (layer B.Cu) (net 16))
 (segment (start 125.73 118.11) (end 125.515001 117.895001) (width 0.6) (layer B.Cu) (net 3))
 (segment (start 125.73 118.11) (end 130.175 118.11) (width 0.6) (layer B.Cu) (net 3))
 (segment (start 160.655 79.375) (end 166.37 79.375) (width 0.6) (layer B.Cu) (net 3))
 (segment (start 166.37 79.375) (end 169.965001 82.970001) (width 0.6) (layer B.Cu) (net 3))
 (segment (start 169.965001 82.970001) (end 170.815 83.82) (width 0.6) (layer B.Cu) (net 3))
 (segment (start 153.814977 72.534977) (end 160.655 79.375) (width 0.6) (layer B.Cu) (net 3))
 (segment (start 125.515001 81.494999) (end 134.475023 72.534977) (width 0.6) (layer B.Cu) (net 3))
 (segment (start 134.475023 72.534977) (end 153.814977 72.534977) (width 0.6) (layer B.Cu) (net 3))
 (segment (start 147.885009 94.477061) (end 145.59501 96.76706) (width 0.6) (layer B.Cu) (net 3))
 (segment (start 145.59501 105.22999) (end 144.75 106.075) (width 0.6) (layer B.Cu) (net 3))
 (segment (start 131.953 95.251073) (end 129.115034 92.413107) (width 0.6) (layer B.Cu) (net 3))
 (segment (start 145.59501 96.76706) (end 145.59501 105.22999) (width 0.6) (layer B.Cu) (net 3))
 (segment (start 144.75 106.075) (end 144.145 106.075) (width 0.6) (layer B.Cu) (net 3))
 (segment (start 131.802999 80.649999) (end 141.402069 80.649999) (width 0.6) (layer B.Cu) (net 3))
 (segment (start 129.115034 92.413107) (end 129.115034 83.337964) (width 0.6) (layer B.Cu) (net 3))
 (segment (start 141.402069 80.649999) (end 147.885009 87.132939) (width 0.6) (layer B.Cu) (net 3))
 (segment (start 147.885009 87.132939) (end 147.885009 94.477061) (width 0.6) (layer B.Cu) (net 3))
 (segment (start 129.115034 83.337964) (end 131.802999 80.649999) (width 0.6) (layer B.Cu) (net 3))
 (segment (start 125.515001 117.895001) (end 125.515001 81.494999) (width 0.6) (layer B.Cu) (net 3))
 (segment (start 130.479999 104.908001) (end 130.479999 100.660001) (width 0.6) (layer B.Cu) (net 3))
 (segment (start 130.479999 100.660001) (end 131.380001 99.759999) (width 0.6) (layer B.Cu) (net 3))
 (segment (start 131.380001 99.759999) (end 132.08 99.06) (width 0.6) (layer B.Cu) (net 3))
 (segment (start 132.543002 106.045) (end 131.616998 106.045) (width 0.6) (layer B.Cu) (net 3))
 (segment (start 131.616998 106.045) (end 130.479999 104.908001) (width 0.6) (layer B.Cu) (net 3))
 (segment (start 135.255 91.895) (end 135.255 103.333002) (width 0.6) (layer B.Cu) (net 3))
 (segment (start 135.255 103.333002) (end 132.543002 106.045) (width 0.6) (layer B.Cu) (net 3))
 (segment (start 137.795 90.805) (end 136.345 90.805) (width 0.6) (layer B.Cu) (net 3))
 (segment (start 136.345 90.805) (end 135.255 91.895) (width 0.6) (layer B.Cu) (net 3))
 (segment (start 132.08 96.266) (end 132.08 99.06) (width 0.6) (layer B.Cu) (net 3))
 (segment (start 132.08 99.06) (end 132.08 98.425) (width 0.6) (layer F.Cu) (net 3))
 (segment (start 144.145 106.075) (end 144.145 108.535623) (width 0.6) (layer B.Cu) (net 3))
 (segment (start 144.145 108.535623) (end 148.639377 113.03) (width 0.6) (layer B.Cu) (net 3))
 (segment (start 148.639377 113.03) (end 149.095 113.03) (width 0.6) (layer B.Cu) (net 3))
 (segment (start 149.095 113.03) (end 150.495 113.03) (width 0.6) (layer B.Cu) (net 3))
 (segment (start 175.045001 104.354999) (end 175.895 103.505) (width 0.6) (layer B.Cu) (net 3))
 (segment (start 174.675999 104.724001) (end 175.045001 104.354999) (width 0.6) (layer B.Cu) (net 3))
 (segment (start 168.859001 104.724001) (end 174.675999 104.724001) (width 0.6) (layer B.Cu) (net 3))
 (segment (start 178.845012 102.205988) (end 177.546 103.505) (width 0.6) (layer B.Cu) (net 3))
 (segment (start 177.546 103.505) (end 175.895 103.505) (width 0.6) (layer B.Cu) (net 3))
 (segment (start 177.465001 82.069999) (end 178.845012 83.45001) (width 0.6) (layer B.Cu) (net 3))
 (segment (start 172.565001 82.069999) (end 177.465001 82.069999) (width 0.6) (layer B.Cu) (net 3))
 (segment (start 178.845012 83.45001) (end 178.845012 102.205988) (width 0.6) (layer B.Cu) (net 3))
 (segment (start 170.815 83.82) (end 172.565001 82.069999) (width 0.6) (layer B.Cu) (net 3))
 (segment (start 165.343 117.704) (end 166.243 117.704) (width 0.6) (layer B.Cu) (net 3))
 (segment (start 158.968999 111.329999) (end 165.343 117.704) (width 0.6) (layer B.Cu) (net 3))
 (segment (start 166.243 109.804) (end 167.64 108.407) (width 0.6) (layer B.Cu) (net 3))
 (segment (start 167.64 108.407) (end 167.64 104.494949) (width 0.6) (layer B.Cu) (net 3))
 (segment (start 166.243 111.404) (end 166.243 109.804) (width 0.6) (layer B.Cu) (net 3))
 (segment (start 150.495 111.63) (end 150.795001 111.329999) (width 0.6) (layer B.Cu) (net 3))
 (segment (start 150.495 113.03) (end 150.495 111.63) (width 0.6) (layer B.Cu) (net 3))
 (segment (start 150.795001 111.329999) (end 158.968999 111.329999) (width 0.6) (layer B.Cu) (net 3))
 (segment (start 167.64 103.505) (end 168.859001 104.724001) (width 0.6) (layer B.Cu) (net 3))
 (segment (start 167.767 100.076) (end 167.767 103.378) (width 0.6) (layer B.Cu) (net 3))
 (segment (start 167.767 103.378) (end 167.64 103.505) (width 0.6) (layer B.Cu) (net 3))
 (segment (start 167.64 104.494949) (end 167.64 103.505) (width 0.6) (layer B.Cu) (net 3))
 (segment (start 158.145 94.075) (end 159.595623 94.075) (width 0.6) (layer B.Cu) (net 9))
 (segment (start 159.595623 94.075) (end 168.275 85.395623) (width 0.6) (layer B.Cu) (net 9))
 (segment (start 168.275 85.395623) (end 168.275 85.022081) (width 0.6) (layer B.Cu) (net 9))
 (segment (start 168.275 85.022081) (end 168.275 83.82) (width 0.6) (layer B.Cu) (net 9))
 (segment (start 158.145 92.075) (end 158.145 91.41) (width 0.6) (layer B.Cu) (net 10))
 (segment (start 158.145 91.41) (end 165.735 83.82) (width 0.6) (layer B.Cu) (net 10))
 (segment (start 129.985 126.285) (end 131.084999 125.185001) (width 0.6) (layer B.Cu) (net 12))
 (segment (start 131.084999 125.185001) (end 134.949999 125.185001) (width 0.6) (layer B.Cu) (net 12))
 (segment (start 134.949999 125.185001) (end 134.989999 125.145001) (width 0.6) (layer B.Cu) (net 12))
 (segment (start 134.989999 125.145001) (end 167.457001 125.145001) (width 0.6) (layer B.Cu) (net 12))
 (segment (start 167.457001 125.145001) (end 176.958001 115.644001) (width 0.6) (layer B.Cu) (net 12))
 (segment (start 176.958001 115.644001) (end 176.958001 112.568001) (width 0.6) (layer B.Cu) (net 12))
 (segment (start 176.958001 112.568001) (end 176.658 112.268) (width 0.6) (layer B.Cu) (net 12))
 (segment (start 176.658 112.268) (end 175.133 112.268) (width 0.6) (layer B.Cu) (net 12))
 (segment (start 135.255 124.88) (end 135.255 118.11) (width 0.6) (layer B.Cu) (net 12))
 (segment (start 168.543 111.404) (end 174.269 111.404) (width 0.6) (layer B.Cu) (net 12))
 (segment (start 174.269 111.404) (end 175.133 112.268) (width 0.6) (layer B.Cu) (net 12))
 (segment (start 140.214999 88.144999) (end 144.145 92.075) (width 0.6) (layer B.Cu) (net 15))
 (segment (start 140.214999 88.049999) (end 140.214999 88.144999) (width 0.6) (layer B.Cu) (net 15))
 (segment (start 139.215 87.05) (end 140.214999 88.049999) (width 0.6) (layer B.Cu) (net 15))
 (segment (start 132.715 88.464213) (end 132.715 87.05) (width 0.6) (layer B.Cu) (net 15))
 (segment (start 131.953 91.186) (end 132.715 90.424) (width 0.6) (layer B.Cu) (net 15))
 (segment (start 132.715 90.424) (end 132.715 88.464213) (width 0.6) (layer B.Cu) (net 15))
 (segment (start 144.145 95.885) (end 144.145 96.075) (width 0.6) (layer B.Cu) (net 17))
 (segment (start 142.870001 84.450001) (end 145.595001 87.175001) (width 0.6) (layer B.Cu) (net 17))
 (segment (start 144.50499 95.52501) (end 144.145 95.885) (width 0.6) (layer B.Cu) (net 17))
 (segment (start 145.595001 95.069999) (end 145.13999 95.52501) (width 0.6) (layer B.Cu) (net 17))
 (segment (start 130.315045 84.949955) (end 130.814999 84.450001) (width 0.6) (layer B.Cu) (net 17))
 (segment (start 130.315045 91.789047) (end 130.315045 84.949955) (width 0.6) (layer B.Cu) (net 17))
 (segment (start 133.985 95.459002) (end 130.315045 91.789047) (width 0.6) (layer B.Cu) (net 17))
 (segment (start 132.08 104.14) (end 133.985 102.235) (width 0.6) (layer B.Cu) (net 17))
 (segment (start 133.985 102.235) (end 133.985 95.459002) (width 0.6) (layer B.Cu) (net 17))
 (segment (start 130.814999 84.450001) (end 142.870001 84.450001) (width 0.6) (layer B.Cu) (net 17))
 (segment (start 145.595001 87.175001) (end 145.595001 95.069999) (width 0.6) (layer B.Cu) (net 17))
 (segment (start 145.13999 95.52501) (end 144.50499 95.52501) (width 0.6) (layer B.Cu) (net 17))
 (segment (start 142.694377 96.075) (end 144.145 96.075) (width 0.6) (layer B.Cu) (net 17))
 (segment (start 144.195623 96.075) (end 144.145 96.075) (width 0.6) (layer B.Cu) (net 17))
 (segment (start 163.328001 105.105001) (end 164.839988 103.593014) (width 0.6) (layer B.Cu) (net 13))
 (segment (start 161.791999 105.105001) (end 163.328001 105.105001) (width 0.6) (layer B.Cu) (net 13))
 (segment (start 160.761998 104.075) (end 161.791999 105.105001) (width 0.6) (layer B.Cu) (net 13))
 (segment (start 171.131001 97.344001) (end 171.831 98.044) (width 0.6) (layer B.Cu) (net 13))
 (segment (start 170.122989 96.335989) (end 171.131001 97.344001) (width 0.6) (layer B.Cu) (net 13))
 (segment (start 167.441938 96.335989) (end 170.122989 96.335989) (width 0.6) (layer B.Cu) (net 13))
 (segment (start 164.839988 98.937939) (end 167.441938 96.335989) (width 0.6) (layer B.Cu) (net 13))
 (segment (start 164.839988 103.593014) (end 164.839988 98.937939) (width 0.6) (layer B.Cu) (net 13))
 (segment (start 158.145 104.075) (end 160.761998 104.075) (width 0.6) (layer B.Cu) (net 13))
 (segment (start 150.395045 96.166045) (end 154.304 100.075) (width 0.6) (layer B.Cu) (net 4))
 (segment (start 158.145 100.075) (end 162.686 100.075) (width 0.6) (layer B.Cu) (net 4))
 (segment (start 162.686 100.075) (end 162.687 100.076) (width 0.6) (layer B.Cu) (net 4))
 (segment (start 154.304 100.075) (end 158.145 100.075) (width 0.6) (layer B.Cu) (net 4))
 (segment (start 151.28 76.835) (end 149.379999 78.735001) (width 0.6) (layer B.Cu) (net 4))
 (segment (start 150.395045 86.248833) (end 150.395045 96.166045) (width 0.6) (layer B.Cu) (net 4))
 (segment (start 149.379999 78.735001) (end 149.379999 85.233787) (width 0.6) (layer B.Cu) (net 4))
 (segment (start 149.379999 85.233787) (end 150.395045 86.248833) (width 0.6) (layer B.Cu) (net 4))
 (segment (start 158.145 102.075) (end 161.13 102.075) (width 0.6) (layer B.Cu) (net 14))
 (segment (start 161.13 102.075) (end 162.56 103.505) (width 0.6) (layer B.Cu) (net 14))
 (segment (start 159.385 131.485) (end 172.045 131.485) (width 2.5) (layer B.Cu) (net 1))
 (segment (start 172.045 131.485) (end 172.085 131.445) (width 0.6) (layer B.Cu) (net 1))
 (segment (start 159.385 136.485) (end 172.045 136.485) (width 2.5) (layer B.Cu) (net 2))
 (segment (start 172.045 136.485) (end 172.085 136.525) (width 0.6) (layer B.Cu) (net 2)))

